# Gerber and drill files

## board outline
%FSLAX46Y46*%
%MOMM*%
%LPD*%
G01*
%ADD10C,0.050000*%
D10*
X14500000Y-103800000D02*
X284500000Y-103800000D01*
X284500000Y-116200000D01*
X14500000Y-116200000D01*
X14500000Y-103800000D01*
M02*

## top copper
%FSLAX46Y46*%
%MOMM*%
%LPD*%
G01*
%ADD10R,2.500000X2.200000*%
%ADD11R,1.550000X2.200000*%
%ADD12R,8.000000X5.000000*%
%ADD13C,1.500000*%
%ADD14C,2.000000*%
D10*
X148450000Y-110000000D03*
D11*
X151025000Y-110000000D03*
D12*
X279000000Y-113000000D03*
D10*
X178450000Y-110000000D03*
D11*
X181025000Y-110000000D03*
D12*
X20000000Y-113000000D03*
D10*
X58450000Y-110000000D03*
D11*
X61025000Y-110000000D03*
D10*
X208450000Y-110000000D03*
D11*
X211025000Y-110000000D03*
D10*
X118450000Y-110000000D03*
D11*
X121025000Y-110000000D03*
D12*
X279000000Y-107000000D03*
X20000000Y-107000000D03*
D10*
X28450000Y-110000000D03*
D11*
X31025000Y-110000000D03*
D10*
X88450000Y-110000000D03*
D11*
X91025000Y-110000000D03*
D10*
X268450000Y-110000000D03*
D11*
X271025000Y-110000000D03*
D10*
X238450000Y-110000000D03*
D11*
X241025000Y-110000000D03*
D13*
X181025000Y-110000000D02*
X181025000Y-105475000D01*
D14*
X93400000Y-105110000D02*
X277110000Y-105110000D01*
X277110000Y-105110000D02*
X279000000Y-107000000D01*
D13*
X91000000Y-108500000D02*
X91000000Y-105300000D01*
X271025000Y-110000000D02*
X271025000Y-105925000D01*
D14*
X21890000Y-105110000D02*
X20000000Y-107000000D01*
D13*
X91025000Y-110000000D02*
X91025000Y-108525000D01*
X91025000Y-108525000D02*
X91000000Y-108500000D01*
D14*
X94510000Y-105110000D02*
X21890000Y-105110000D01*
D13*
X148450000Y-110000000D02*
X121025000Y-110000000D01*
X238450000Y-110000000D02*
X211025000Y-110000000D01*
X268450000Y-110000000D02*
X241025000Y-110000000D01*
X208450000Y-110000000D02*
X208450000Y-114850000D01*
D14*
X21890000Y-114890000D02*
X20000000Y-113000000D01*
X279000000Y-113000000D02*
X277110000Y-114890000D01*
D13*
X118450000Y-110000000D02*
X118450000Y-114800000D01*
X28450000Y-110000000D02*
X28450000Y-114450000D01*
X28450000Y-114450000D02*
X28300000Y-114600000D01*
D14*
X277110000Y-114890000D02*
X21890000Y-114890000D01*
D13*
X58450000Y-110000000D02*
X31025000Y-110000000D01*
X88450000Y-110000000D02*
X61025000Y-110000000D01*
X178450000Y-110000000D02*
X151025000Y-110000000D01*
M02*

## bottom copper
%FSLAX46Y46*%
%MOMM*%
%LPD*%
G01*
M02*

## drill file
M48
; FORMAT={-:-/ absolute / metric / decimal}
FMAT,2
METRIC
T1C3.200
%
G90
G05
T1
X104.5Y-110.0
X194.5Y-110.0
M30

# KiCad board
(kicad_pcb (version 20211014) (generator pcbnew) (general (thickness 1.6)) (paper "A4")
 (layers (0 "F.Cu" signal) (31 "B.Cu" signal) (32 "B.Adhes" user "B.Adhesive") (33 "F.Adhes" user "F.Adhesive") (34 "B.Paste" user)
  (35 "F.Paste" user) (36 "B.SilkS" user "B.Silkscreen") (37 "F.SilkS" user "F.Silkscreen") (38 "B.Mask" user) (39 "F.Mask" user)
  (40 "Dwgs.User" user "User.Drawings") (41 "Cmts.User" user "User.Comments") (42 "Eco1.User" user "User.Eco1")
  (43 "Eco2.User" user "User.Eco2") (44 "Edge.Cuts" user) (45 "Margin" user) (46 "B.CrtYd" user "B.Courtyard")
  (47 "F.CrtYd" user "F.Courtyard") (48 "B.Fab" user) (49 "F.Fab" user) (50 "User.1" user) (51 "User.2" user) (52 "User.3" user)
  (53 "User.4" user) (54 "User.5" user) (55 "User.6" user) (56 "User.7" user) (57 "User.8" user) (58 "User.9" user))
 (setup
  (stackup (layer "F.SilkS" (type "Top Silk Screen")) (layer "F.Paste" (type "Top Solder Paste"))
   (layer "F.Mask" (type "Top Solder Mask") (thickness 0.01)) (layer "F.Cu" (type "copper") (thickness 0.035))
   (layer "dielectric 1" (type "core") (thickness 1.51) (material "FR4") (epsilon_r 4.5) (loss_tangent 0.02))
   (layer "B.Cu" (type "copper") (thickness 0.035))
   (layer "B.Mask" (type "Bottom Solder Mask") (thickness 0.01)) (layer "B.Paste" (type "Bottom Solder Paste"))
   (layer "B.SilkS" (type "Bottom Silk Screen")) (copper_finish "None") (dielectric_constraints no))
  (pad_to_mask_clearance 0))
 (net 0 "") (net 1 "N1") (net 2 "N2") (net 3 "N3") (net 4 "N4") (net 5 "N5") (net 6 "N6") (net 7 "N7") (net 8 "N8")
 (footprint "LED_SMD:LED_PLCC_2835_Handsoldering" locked (layer "F.Cu") (at 149.5 110)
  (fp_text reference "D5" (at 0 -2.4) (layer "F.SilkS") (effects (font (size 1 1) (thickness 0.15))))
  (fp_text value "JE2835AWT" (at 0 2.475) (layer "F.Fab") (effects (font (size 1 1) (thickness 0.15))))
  (pad "1" smd rect locked (at -1.05 0) (size 2.5 2.2) (layers "F.Cu" "F.Paste" "F.Mask") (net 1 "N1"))
  (pad "2" smd rect locked (at 1.525 0) (size 1.55 2.2) (layers "F.Cu" "F.Paste" "F.Mask") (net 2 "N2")))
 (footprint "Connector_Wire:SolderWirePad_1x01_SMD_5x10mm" (layer "F.Cu") (at 278.6 113 -90)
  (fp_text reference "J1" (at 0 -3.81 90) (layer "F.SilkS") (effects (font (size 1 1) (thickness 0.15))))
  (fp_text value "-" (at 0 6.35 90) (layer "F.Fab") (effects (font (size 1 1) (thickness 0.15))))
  (pad "1" smd rect locked (at 0 -0.4 270) (size 5 8) (layers "F.Cu" "F.Paste" "F.Mask") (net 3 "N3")))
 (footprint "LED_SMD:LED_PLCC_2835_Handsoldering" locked (layer "F.Cu") (at 179.5 110)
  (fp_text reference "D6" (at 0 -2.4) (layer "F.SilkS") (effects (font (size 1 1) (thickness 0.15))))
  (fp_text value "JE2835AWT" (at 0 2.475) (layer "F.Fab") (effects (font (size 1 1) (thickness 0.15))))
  (pad "1" smd rect locked (at -1.05 0) (size 2.5 2.2) (layers "F.Cu" "F.Paste" "F.Mask") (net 2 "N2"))
  (pad "2" smd rect locked (at 1.525 0) (size 1.55 2.2) (layers "F.Cu" "F.Paste" "F.Mask") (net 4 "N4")))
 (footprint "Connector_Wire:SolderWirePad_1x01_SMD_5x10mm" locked (layer "F.Cu") (at 20 112 90)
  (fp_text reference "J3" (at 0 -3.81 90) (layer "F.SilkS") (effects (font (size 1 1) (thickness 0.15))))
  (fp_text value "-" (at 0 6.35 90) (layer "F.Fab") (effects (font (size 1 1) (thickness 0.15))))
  (pad "1" smd rect locked (at -1 0 90) (size 5 8) (layers "F.Cu" "F.Paste" "F.Mask") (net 3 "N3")))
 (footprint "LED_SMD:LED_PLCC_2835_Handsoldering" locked (layer "F.Cu") (at 59.5 110)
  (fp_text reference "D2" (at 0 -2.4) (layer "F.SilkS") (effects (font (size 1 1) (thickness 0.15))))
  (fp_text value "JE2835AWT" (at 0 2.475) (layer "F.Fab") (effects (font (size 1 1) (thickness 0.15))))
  (pad "1" smd rect locked (at -1.05 0) (size 2.5 2.2) (layers "F.Cu" "F.Paste" "F.Mask") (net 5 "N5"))
  (pad "2" smd rect locked (at 1.525 0) (size 1.55 2.2) (layers "F.Cu" "F.Paste" "F.Mask") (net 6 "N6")))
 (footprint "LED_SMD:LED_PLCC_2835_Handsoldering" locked (layer "F.Cu") (at 209.5 110)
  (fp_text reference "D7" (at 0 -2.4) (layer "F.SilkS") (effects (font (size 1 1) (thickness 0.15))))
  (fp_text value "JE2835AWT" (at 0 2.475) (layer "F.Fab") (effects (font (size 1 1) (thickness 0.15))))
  (pad "1" smd rect locked (at -1.05 0) (size 2.5 2.2) (layers "F.Cu" "F.Paste" "F.Mask") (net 3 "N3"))
  (pad "2" smd rect locked (at 1.525 0) (size 1.55 2.2) (layers "F.Cu" "F.Paste" "F.Mask") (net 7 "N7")))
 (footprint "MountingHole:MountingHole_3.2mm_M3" (layer "F.Cu") (at 194.5 110)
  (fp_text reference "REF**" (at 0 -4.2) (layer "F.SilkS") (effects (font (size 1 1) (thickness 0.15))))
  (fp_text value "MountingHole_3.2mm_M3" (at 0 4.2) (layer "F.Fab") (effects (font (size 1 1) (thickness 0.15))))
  (pad "" np_thru_hole circle (at 0 0) (size 3.2 3.2) (drill 3.2) (layers *.Cu *.Mask)))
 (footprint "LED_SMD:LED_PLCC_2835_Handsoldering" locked (layer "F.Cu") (at 119.5 110)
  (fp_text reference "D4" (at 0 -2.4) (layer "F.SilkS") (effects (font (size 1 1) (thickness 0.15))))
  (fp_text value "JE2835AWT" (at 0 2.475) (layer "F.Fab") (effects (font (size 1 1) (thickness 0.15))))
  (pad "1" smd rect locked (at -1.05 0) (size 2.5 2.2) (layers "F.Cu" "F.Paste" "F.Mask") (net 3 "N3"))
  (pad "2" smd rect locked (at 1.525 0) (size 1.55 2.2) (layers "F.Cu" "F.Paste" "F.Mask") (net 1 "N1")))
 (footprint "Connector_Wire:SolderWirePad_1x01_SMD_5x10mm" (layer "F.Cu") (at 278.6 108 -90)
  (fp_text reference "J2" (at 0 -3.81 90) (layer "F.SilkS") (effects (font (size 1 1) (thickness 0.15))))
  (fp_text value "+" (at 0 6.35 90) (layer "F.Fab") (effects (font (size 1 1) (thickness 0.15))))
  (pad "1" smd rect locked (at -1 -0.4 270) (size 5 8) (layers "F.Cu" "F.Paste" "F.Mask") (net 4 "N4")))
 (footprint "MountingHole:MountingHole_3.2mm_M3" (layer "F.Cu") (at 104.5 110)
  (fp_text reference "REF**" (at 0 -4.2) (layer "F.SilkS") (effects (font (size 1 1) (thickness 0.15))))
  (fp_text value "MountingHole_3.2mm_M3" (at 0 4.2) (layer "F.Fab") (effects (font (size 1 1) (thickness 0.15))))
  (pad "" np_thru_hole circle (at 0 0) (size 3.2 3.2) (drill 3.2) (layers *.Cu *.Mask)))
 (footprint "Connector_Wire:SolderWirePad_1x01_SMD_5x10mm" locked (layer "F.Cu") (at 20 108 90)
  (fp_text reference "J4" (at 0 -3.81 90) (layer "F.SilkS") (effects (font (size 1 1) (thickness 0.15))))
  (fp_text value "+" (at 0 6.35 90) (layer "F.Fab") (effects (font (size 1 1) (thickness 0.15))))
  (pad "1" smd rect locked (at 1 0 90) (size 5 8) (layers "F.Cu" "F.Paste" "F.Mask") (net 4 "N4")))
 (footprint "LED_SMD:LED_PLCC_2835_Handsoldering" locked (layer "F.Cu") (at 29.5 110)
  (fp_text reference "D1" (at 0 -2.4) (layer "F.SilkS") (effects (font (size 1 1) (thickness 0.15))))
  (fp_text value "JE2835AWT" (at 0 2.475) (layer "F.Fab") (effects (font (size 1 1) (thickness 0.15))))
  (pad "1" smd rect locked (at -1.05 0) (size 2.5 2.2) (layers "F.Cu" "F.Paste" "F.Mask") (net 3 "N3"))
  (pad "2" smd rect locked (at 1.525 0) (size 1.55 2.2) (layers "F.Cu" "F.Paste" "F.Mask") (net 5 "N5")))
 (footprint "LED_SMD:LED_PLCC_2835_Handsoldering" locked (layer "F.Cu") (at 89.5 110)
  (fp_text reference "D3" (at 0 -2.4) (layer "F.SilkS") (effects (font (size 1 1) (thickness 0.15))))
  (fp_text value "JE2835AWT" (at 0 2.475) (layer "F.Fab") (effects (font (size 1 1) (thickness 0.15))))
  (pad "1" smd rect locked (at -1.05 0) (size 2.5 2.2) (layers "F.Cu" "F.Paste" "F.Mask") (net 6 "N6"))
  (pad "2" smd rect locked (at 1.525 0) (size 1.55 2.2) (layers "F.Cu" "F.Paste" "F.Mask") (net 4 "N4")))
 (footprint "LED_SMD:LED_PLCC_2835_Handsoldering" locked (layer "F.Cu") (at 269.5 110)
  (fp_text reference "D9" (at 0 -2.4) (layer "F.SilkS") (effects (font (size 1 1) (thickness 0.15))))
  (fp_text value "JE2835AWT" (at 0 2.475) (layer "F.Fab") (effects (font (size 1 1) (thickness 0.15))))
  (pad "1" smd rect locked (at -1.05 0) (size 2.5 2.2) (layers "F.Cu" "F.Paste" "F.Mask") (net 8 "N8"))
  (pad "2" smd rect locked (at 1.525 0) (size 1.55 2.2) (layers "F.Cu" "F.Paste" "F.Mask") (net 4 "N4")))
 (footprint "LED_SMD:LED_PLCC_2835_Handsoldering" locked (layer "F.Cu") (at 239.5 110)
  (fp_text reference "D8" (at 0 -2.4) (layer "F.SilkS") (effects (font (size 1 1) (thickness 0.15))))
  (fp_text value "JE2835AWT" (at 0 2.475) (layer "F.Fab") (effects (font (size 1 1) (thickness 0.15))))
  (pad "1" smd rect locked (at -1.05 0) (size 2.5 2.2) (layers "F.Cu" "F.Paste" "F.Mask") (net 7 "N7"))
  (pad "2" smd rect locked (at 1.525 0) (size 1.55 2.2) (layers "F.Cu" "F.Paste" "F.Mask") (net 8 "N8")))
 (gr_rect locked (start 14.5 103.8) (end 284.5 116.2) (layer "Edge.Cuts") (width 0.05) (fill none))
 (segment (start 181.025 110) (end 181.025 105.475) (width 1.5) (layer "F.Cu") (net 4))
 (segment (start 93.4 105.11) (end 277.11 105.11) (width 2) (layer "F.Cu") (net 4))
 (segment (start 277.11 105.11) (end 279 107) (width 2) (layer "F.Cu") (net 4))
 (segment (start 91 108.5) (end 91 105.3) (width 1.5) (layer "F.Cu") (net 4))
 (segment (start 271.025 110) (end 271.025 105.925) (width 1.5) (layer "F.Cu") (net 4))
 (segment (start 21.89 105.11) (end 20 107) (width 2) (layer "F.Cu") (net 4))
 (segment (start 91.025 110) (end 91.025 108.525) (width 1.5) (layer "F.Cu") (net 4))
 (segment (start 91.025 108.525) (end 91 108.5) (width 1.5) (layer "F.Cu") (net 4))
 (segment (start 94.51 105.11) (end 21.89 105.11) (width 2) (layer "F.Cu") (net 4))
 (segment (start 148.45 110) (end 121.025 110) (width 1.5) (layer "F.Cu") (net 1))
 (segment (start 238.45 110) (end 211.025 110) (width 1.5) (layer "F.Cu") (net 7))
 (segment (start 268.45 110) (end 241.025 110) (width 1.5) (layer "F.Cu") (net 8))
 (segment (start 208.45 110) (end 208.45 114.85) (width 1.5) (layer "F.Cu") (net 3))
 (segment (start 21.89 114.89) (end 20 113) (width 2) (layer "F.Cu") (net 3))
 (segment (start 279 113) (end 277.11 114.89) (width 2) (layer "F.Cu") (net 3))
 (segment (start 118.45 110) (end 118.45 114.8) (width 1.5) (layer "F.Cu") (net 3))
 (segment (start 28.45 110) (end 28.45 114.45) (width 1.5) (layer "F.Cu") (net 3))
 (segment (start 28.45 114.45) (end 28.3 114.6) (width 1.5) (layer "F.Cu") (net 3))
 (segment (start 277.11 114.89) (end 21.89 114.89) (width 2) (layer "F.Cu") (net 3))
 (segment (start 58.45 110) (end 31.025 110) (width 1.5) (layer "F.Cu") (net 5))
 (segment (start 88.45 110) (end 61.025 110) (width 1.5) (layer "F.Cu") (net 6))
 (segment (start 178.45 110) (end 151.025 110) (width 1.5) (layer "F.Cu") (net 2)))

